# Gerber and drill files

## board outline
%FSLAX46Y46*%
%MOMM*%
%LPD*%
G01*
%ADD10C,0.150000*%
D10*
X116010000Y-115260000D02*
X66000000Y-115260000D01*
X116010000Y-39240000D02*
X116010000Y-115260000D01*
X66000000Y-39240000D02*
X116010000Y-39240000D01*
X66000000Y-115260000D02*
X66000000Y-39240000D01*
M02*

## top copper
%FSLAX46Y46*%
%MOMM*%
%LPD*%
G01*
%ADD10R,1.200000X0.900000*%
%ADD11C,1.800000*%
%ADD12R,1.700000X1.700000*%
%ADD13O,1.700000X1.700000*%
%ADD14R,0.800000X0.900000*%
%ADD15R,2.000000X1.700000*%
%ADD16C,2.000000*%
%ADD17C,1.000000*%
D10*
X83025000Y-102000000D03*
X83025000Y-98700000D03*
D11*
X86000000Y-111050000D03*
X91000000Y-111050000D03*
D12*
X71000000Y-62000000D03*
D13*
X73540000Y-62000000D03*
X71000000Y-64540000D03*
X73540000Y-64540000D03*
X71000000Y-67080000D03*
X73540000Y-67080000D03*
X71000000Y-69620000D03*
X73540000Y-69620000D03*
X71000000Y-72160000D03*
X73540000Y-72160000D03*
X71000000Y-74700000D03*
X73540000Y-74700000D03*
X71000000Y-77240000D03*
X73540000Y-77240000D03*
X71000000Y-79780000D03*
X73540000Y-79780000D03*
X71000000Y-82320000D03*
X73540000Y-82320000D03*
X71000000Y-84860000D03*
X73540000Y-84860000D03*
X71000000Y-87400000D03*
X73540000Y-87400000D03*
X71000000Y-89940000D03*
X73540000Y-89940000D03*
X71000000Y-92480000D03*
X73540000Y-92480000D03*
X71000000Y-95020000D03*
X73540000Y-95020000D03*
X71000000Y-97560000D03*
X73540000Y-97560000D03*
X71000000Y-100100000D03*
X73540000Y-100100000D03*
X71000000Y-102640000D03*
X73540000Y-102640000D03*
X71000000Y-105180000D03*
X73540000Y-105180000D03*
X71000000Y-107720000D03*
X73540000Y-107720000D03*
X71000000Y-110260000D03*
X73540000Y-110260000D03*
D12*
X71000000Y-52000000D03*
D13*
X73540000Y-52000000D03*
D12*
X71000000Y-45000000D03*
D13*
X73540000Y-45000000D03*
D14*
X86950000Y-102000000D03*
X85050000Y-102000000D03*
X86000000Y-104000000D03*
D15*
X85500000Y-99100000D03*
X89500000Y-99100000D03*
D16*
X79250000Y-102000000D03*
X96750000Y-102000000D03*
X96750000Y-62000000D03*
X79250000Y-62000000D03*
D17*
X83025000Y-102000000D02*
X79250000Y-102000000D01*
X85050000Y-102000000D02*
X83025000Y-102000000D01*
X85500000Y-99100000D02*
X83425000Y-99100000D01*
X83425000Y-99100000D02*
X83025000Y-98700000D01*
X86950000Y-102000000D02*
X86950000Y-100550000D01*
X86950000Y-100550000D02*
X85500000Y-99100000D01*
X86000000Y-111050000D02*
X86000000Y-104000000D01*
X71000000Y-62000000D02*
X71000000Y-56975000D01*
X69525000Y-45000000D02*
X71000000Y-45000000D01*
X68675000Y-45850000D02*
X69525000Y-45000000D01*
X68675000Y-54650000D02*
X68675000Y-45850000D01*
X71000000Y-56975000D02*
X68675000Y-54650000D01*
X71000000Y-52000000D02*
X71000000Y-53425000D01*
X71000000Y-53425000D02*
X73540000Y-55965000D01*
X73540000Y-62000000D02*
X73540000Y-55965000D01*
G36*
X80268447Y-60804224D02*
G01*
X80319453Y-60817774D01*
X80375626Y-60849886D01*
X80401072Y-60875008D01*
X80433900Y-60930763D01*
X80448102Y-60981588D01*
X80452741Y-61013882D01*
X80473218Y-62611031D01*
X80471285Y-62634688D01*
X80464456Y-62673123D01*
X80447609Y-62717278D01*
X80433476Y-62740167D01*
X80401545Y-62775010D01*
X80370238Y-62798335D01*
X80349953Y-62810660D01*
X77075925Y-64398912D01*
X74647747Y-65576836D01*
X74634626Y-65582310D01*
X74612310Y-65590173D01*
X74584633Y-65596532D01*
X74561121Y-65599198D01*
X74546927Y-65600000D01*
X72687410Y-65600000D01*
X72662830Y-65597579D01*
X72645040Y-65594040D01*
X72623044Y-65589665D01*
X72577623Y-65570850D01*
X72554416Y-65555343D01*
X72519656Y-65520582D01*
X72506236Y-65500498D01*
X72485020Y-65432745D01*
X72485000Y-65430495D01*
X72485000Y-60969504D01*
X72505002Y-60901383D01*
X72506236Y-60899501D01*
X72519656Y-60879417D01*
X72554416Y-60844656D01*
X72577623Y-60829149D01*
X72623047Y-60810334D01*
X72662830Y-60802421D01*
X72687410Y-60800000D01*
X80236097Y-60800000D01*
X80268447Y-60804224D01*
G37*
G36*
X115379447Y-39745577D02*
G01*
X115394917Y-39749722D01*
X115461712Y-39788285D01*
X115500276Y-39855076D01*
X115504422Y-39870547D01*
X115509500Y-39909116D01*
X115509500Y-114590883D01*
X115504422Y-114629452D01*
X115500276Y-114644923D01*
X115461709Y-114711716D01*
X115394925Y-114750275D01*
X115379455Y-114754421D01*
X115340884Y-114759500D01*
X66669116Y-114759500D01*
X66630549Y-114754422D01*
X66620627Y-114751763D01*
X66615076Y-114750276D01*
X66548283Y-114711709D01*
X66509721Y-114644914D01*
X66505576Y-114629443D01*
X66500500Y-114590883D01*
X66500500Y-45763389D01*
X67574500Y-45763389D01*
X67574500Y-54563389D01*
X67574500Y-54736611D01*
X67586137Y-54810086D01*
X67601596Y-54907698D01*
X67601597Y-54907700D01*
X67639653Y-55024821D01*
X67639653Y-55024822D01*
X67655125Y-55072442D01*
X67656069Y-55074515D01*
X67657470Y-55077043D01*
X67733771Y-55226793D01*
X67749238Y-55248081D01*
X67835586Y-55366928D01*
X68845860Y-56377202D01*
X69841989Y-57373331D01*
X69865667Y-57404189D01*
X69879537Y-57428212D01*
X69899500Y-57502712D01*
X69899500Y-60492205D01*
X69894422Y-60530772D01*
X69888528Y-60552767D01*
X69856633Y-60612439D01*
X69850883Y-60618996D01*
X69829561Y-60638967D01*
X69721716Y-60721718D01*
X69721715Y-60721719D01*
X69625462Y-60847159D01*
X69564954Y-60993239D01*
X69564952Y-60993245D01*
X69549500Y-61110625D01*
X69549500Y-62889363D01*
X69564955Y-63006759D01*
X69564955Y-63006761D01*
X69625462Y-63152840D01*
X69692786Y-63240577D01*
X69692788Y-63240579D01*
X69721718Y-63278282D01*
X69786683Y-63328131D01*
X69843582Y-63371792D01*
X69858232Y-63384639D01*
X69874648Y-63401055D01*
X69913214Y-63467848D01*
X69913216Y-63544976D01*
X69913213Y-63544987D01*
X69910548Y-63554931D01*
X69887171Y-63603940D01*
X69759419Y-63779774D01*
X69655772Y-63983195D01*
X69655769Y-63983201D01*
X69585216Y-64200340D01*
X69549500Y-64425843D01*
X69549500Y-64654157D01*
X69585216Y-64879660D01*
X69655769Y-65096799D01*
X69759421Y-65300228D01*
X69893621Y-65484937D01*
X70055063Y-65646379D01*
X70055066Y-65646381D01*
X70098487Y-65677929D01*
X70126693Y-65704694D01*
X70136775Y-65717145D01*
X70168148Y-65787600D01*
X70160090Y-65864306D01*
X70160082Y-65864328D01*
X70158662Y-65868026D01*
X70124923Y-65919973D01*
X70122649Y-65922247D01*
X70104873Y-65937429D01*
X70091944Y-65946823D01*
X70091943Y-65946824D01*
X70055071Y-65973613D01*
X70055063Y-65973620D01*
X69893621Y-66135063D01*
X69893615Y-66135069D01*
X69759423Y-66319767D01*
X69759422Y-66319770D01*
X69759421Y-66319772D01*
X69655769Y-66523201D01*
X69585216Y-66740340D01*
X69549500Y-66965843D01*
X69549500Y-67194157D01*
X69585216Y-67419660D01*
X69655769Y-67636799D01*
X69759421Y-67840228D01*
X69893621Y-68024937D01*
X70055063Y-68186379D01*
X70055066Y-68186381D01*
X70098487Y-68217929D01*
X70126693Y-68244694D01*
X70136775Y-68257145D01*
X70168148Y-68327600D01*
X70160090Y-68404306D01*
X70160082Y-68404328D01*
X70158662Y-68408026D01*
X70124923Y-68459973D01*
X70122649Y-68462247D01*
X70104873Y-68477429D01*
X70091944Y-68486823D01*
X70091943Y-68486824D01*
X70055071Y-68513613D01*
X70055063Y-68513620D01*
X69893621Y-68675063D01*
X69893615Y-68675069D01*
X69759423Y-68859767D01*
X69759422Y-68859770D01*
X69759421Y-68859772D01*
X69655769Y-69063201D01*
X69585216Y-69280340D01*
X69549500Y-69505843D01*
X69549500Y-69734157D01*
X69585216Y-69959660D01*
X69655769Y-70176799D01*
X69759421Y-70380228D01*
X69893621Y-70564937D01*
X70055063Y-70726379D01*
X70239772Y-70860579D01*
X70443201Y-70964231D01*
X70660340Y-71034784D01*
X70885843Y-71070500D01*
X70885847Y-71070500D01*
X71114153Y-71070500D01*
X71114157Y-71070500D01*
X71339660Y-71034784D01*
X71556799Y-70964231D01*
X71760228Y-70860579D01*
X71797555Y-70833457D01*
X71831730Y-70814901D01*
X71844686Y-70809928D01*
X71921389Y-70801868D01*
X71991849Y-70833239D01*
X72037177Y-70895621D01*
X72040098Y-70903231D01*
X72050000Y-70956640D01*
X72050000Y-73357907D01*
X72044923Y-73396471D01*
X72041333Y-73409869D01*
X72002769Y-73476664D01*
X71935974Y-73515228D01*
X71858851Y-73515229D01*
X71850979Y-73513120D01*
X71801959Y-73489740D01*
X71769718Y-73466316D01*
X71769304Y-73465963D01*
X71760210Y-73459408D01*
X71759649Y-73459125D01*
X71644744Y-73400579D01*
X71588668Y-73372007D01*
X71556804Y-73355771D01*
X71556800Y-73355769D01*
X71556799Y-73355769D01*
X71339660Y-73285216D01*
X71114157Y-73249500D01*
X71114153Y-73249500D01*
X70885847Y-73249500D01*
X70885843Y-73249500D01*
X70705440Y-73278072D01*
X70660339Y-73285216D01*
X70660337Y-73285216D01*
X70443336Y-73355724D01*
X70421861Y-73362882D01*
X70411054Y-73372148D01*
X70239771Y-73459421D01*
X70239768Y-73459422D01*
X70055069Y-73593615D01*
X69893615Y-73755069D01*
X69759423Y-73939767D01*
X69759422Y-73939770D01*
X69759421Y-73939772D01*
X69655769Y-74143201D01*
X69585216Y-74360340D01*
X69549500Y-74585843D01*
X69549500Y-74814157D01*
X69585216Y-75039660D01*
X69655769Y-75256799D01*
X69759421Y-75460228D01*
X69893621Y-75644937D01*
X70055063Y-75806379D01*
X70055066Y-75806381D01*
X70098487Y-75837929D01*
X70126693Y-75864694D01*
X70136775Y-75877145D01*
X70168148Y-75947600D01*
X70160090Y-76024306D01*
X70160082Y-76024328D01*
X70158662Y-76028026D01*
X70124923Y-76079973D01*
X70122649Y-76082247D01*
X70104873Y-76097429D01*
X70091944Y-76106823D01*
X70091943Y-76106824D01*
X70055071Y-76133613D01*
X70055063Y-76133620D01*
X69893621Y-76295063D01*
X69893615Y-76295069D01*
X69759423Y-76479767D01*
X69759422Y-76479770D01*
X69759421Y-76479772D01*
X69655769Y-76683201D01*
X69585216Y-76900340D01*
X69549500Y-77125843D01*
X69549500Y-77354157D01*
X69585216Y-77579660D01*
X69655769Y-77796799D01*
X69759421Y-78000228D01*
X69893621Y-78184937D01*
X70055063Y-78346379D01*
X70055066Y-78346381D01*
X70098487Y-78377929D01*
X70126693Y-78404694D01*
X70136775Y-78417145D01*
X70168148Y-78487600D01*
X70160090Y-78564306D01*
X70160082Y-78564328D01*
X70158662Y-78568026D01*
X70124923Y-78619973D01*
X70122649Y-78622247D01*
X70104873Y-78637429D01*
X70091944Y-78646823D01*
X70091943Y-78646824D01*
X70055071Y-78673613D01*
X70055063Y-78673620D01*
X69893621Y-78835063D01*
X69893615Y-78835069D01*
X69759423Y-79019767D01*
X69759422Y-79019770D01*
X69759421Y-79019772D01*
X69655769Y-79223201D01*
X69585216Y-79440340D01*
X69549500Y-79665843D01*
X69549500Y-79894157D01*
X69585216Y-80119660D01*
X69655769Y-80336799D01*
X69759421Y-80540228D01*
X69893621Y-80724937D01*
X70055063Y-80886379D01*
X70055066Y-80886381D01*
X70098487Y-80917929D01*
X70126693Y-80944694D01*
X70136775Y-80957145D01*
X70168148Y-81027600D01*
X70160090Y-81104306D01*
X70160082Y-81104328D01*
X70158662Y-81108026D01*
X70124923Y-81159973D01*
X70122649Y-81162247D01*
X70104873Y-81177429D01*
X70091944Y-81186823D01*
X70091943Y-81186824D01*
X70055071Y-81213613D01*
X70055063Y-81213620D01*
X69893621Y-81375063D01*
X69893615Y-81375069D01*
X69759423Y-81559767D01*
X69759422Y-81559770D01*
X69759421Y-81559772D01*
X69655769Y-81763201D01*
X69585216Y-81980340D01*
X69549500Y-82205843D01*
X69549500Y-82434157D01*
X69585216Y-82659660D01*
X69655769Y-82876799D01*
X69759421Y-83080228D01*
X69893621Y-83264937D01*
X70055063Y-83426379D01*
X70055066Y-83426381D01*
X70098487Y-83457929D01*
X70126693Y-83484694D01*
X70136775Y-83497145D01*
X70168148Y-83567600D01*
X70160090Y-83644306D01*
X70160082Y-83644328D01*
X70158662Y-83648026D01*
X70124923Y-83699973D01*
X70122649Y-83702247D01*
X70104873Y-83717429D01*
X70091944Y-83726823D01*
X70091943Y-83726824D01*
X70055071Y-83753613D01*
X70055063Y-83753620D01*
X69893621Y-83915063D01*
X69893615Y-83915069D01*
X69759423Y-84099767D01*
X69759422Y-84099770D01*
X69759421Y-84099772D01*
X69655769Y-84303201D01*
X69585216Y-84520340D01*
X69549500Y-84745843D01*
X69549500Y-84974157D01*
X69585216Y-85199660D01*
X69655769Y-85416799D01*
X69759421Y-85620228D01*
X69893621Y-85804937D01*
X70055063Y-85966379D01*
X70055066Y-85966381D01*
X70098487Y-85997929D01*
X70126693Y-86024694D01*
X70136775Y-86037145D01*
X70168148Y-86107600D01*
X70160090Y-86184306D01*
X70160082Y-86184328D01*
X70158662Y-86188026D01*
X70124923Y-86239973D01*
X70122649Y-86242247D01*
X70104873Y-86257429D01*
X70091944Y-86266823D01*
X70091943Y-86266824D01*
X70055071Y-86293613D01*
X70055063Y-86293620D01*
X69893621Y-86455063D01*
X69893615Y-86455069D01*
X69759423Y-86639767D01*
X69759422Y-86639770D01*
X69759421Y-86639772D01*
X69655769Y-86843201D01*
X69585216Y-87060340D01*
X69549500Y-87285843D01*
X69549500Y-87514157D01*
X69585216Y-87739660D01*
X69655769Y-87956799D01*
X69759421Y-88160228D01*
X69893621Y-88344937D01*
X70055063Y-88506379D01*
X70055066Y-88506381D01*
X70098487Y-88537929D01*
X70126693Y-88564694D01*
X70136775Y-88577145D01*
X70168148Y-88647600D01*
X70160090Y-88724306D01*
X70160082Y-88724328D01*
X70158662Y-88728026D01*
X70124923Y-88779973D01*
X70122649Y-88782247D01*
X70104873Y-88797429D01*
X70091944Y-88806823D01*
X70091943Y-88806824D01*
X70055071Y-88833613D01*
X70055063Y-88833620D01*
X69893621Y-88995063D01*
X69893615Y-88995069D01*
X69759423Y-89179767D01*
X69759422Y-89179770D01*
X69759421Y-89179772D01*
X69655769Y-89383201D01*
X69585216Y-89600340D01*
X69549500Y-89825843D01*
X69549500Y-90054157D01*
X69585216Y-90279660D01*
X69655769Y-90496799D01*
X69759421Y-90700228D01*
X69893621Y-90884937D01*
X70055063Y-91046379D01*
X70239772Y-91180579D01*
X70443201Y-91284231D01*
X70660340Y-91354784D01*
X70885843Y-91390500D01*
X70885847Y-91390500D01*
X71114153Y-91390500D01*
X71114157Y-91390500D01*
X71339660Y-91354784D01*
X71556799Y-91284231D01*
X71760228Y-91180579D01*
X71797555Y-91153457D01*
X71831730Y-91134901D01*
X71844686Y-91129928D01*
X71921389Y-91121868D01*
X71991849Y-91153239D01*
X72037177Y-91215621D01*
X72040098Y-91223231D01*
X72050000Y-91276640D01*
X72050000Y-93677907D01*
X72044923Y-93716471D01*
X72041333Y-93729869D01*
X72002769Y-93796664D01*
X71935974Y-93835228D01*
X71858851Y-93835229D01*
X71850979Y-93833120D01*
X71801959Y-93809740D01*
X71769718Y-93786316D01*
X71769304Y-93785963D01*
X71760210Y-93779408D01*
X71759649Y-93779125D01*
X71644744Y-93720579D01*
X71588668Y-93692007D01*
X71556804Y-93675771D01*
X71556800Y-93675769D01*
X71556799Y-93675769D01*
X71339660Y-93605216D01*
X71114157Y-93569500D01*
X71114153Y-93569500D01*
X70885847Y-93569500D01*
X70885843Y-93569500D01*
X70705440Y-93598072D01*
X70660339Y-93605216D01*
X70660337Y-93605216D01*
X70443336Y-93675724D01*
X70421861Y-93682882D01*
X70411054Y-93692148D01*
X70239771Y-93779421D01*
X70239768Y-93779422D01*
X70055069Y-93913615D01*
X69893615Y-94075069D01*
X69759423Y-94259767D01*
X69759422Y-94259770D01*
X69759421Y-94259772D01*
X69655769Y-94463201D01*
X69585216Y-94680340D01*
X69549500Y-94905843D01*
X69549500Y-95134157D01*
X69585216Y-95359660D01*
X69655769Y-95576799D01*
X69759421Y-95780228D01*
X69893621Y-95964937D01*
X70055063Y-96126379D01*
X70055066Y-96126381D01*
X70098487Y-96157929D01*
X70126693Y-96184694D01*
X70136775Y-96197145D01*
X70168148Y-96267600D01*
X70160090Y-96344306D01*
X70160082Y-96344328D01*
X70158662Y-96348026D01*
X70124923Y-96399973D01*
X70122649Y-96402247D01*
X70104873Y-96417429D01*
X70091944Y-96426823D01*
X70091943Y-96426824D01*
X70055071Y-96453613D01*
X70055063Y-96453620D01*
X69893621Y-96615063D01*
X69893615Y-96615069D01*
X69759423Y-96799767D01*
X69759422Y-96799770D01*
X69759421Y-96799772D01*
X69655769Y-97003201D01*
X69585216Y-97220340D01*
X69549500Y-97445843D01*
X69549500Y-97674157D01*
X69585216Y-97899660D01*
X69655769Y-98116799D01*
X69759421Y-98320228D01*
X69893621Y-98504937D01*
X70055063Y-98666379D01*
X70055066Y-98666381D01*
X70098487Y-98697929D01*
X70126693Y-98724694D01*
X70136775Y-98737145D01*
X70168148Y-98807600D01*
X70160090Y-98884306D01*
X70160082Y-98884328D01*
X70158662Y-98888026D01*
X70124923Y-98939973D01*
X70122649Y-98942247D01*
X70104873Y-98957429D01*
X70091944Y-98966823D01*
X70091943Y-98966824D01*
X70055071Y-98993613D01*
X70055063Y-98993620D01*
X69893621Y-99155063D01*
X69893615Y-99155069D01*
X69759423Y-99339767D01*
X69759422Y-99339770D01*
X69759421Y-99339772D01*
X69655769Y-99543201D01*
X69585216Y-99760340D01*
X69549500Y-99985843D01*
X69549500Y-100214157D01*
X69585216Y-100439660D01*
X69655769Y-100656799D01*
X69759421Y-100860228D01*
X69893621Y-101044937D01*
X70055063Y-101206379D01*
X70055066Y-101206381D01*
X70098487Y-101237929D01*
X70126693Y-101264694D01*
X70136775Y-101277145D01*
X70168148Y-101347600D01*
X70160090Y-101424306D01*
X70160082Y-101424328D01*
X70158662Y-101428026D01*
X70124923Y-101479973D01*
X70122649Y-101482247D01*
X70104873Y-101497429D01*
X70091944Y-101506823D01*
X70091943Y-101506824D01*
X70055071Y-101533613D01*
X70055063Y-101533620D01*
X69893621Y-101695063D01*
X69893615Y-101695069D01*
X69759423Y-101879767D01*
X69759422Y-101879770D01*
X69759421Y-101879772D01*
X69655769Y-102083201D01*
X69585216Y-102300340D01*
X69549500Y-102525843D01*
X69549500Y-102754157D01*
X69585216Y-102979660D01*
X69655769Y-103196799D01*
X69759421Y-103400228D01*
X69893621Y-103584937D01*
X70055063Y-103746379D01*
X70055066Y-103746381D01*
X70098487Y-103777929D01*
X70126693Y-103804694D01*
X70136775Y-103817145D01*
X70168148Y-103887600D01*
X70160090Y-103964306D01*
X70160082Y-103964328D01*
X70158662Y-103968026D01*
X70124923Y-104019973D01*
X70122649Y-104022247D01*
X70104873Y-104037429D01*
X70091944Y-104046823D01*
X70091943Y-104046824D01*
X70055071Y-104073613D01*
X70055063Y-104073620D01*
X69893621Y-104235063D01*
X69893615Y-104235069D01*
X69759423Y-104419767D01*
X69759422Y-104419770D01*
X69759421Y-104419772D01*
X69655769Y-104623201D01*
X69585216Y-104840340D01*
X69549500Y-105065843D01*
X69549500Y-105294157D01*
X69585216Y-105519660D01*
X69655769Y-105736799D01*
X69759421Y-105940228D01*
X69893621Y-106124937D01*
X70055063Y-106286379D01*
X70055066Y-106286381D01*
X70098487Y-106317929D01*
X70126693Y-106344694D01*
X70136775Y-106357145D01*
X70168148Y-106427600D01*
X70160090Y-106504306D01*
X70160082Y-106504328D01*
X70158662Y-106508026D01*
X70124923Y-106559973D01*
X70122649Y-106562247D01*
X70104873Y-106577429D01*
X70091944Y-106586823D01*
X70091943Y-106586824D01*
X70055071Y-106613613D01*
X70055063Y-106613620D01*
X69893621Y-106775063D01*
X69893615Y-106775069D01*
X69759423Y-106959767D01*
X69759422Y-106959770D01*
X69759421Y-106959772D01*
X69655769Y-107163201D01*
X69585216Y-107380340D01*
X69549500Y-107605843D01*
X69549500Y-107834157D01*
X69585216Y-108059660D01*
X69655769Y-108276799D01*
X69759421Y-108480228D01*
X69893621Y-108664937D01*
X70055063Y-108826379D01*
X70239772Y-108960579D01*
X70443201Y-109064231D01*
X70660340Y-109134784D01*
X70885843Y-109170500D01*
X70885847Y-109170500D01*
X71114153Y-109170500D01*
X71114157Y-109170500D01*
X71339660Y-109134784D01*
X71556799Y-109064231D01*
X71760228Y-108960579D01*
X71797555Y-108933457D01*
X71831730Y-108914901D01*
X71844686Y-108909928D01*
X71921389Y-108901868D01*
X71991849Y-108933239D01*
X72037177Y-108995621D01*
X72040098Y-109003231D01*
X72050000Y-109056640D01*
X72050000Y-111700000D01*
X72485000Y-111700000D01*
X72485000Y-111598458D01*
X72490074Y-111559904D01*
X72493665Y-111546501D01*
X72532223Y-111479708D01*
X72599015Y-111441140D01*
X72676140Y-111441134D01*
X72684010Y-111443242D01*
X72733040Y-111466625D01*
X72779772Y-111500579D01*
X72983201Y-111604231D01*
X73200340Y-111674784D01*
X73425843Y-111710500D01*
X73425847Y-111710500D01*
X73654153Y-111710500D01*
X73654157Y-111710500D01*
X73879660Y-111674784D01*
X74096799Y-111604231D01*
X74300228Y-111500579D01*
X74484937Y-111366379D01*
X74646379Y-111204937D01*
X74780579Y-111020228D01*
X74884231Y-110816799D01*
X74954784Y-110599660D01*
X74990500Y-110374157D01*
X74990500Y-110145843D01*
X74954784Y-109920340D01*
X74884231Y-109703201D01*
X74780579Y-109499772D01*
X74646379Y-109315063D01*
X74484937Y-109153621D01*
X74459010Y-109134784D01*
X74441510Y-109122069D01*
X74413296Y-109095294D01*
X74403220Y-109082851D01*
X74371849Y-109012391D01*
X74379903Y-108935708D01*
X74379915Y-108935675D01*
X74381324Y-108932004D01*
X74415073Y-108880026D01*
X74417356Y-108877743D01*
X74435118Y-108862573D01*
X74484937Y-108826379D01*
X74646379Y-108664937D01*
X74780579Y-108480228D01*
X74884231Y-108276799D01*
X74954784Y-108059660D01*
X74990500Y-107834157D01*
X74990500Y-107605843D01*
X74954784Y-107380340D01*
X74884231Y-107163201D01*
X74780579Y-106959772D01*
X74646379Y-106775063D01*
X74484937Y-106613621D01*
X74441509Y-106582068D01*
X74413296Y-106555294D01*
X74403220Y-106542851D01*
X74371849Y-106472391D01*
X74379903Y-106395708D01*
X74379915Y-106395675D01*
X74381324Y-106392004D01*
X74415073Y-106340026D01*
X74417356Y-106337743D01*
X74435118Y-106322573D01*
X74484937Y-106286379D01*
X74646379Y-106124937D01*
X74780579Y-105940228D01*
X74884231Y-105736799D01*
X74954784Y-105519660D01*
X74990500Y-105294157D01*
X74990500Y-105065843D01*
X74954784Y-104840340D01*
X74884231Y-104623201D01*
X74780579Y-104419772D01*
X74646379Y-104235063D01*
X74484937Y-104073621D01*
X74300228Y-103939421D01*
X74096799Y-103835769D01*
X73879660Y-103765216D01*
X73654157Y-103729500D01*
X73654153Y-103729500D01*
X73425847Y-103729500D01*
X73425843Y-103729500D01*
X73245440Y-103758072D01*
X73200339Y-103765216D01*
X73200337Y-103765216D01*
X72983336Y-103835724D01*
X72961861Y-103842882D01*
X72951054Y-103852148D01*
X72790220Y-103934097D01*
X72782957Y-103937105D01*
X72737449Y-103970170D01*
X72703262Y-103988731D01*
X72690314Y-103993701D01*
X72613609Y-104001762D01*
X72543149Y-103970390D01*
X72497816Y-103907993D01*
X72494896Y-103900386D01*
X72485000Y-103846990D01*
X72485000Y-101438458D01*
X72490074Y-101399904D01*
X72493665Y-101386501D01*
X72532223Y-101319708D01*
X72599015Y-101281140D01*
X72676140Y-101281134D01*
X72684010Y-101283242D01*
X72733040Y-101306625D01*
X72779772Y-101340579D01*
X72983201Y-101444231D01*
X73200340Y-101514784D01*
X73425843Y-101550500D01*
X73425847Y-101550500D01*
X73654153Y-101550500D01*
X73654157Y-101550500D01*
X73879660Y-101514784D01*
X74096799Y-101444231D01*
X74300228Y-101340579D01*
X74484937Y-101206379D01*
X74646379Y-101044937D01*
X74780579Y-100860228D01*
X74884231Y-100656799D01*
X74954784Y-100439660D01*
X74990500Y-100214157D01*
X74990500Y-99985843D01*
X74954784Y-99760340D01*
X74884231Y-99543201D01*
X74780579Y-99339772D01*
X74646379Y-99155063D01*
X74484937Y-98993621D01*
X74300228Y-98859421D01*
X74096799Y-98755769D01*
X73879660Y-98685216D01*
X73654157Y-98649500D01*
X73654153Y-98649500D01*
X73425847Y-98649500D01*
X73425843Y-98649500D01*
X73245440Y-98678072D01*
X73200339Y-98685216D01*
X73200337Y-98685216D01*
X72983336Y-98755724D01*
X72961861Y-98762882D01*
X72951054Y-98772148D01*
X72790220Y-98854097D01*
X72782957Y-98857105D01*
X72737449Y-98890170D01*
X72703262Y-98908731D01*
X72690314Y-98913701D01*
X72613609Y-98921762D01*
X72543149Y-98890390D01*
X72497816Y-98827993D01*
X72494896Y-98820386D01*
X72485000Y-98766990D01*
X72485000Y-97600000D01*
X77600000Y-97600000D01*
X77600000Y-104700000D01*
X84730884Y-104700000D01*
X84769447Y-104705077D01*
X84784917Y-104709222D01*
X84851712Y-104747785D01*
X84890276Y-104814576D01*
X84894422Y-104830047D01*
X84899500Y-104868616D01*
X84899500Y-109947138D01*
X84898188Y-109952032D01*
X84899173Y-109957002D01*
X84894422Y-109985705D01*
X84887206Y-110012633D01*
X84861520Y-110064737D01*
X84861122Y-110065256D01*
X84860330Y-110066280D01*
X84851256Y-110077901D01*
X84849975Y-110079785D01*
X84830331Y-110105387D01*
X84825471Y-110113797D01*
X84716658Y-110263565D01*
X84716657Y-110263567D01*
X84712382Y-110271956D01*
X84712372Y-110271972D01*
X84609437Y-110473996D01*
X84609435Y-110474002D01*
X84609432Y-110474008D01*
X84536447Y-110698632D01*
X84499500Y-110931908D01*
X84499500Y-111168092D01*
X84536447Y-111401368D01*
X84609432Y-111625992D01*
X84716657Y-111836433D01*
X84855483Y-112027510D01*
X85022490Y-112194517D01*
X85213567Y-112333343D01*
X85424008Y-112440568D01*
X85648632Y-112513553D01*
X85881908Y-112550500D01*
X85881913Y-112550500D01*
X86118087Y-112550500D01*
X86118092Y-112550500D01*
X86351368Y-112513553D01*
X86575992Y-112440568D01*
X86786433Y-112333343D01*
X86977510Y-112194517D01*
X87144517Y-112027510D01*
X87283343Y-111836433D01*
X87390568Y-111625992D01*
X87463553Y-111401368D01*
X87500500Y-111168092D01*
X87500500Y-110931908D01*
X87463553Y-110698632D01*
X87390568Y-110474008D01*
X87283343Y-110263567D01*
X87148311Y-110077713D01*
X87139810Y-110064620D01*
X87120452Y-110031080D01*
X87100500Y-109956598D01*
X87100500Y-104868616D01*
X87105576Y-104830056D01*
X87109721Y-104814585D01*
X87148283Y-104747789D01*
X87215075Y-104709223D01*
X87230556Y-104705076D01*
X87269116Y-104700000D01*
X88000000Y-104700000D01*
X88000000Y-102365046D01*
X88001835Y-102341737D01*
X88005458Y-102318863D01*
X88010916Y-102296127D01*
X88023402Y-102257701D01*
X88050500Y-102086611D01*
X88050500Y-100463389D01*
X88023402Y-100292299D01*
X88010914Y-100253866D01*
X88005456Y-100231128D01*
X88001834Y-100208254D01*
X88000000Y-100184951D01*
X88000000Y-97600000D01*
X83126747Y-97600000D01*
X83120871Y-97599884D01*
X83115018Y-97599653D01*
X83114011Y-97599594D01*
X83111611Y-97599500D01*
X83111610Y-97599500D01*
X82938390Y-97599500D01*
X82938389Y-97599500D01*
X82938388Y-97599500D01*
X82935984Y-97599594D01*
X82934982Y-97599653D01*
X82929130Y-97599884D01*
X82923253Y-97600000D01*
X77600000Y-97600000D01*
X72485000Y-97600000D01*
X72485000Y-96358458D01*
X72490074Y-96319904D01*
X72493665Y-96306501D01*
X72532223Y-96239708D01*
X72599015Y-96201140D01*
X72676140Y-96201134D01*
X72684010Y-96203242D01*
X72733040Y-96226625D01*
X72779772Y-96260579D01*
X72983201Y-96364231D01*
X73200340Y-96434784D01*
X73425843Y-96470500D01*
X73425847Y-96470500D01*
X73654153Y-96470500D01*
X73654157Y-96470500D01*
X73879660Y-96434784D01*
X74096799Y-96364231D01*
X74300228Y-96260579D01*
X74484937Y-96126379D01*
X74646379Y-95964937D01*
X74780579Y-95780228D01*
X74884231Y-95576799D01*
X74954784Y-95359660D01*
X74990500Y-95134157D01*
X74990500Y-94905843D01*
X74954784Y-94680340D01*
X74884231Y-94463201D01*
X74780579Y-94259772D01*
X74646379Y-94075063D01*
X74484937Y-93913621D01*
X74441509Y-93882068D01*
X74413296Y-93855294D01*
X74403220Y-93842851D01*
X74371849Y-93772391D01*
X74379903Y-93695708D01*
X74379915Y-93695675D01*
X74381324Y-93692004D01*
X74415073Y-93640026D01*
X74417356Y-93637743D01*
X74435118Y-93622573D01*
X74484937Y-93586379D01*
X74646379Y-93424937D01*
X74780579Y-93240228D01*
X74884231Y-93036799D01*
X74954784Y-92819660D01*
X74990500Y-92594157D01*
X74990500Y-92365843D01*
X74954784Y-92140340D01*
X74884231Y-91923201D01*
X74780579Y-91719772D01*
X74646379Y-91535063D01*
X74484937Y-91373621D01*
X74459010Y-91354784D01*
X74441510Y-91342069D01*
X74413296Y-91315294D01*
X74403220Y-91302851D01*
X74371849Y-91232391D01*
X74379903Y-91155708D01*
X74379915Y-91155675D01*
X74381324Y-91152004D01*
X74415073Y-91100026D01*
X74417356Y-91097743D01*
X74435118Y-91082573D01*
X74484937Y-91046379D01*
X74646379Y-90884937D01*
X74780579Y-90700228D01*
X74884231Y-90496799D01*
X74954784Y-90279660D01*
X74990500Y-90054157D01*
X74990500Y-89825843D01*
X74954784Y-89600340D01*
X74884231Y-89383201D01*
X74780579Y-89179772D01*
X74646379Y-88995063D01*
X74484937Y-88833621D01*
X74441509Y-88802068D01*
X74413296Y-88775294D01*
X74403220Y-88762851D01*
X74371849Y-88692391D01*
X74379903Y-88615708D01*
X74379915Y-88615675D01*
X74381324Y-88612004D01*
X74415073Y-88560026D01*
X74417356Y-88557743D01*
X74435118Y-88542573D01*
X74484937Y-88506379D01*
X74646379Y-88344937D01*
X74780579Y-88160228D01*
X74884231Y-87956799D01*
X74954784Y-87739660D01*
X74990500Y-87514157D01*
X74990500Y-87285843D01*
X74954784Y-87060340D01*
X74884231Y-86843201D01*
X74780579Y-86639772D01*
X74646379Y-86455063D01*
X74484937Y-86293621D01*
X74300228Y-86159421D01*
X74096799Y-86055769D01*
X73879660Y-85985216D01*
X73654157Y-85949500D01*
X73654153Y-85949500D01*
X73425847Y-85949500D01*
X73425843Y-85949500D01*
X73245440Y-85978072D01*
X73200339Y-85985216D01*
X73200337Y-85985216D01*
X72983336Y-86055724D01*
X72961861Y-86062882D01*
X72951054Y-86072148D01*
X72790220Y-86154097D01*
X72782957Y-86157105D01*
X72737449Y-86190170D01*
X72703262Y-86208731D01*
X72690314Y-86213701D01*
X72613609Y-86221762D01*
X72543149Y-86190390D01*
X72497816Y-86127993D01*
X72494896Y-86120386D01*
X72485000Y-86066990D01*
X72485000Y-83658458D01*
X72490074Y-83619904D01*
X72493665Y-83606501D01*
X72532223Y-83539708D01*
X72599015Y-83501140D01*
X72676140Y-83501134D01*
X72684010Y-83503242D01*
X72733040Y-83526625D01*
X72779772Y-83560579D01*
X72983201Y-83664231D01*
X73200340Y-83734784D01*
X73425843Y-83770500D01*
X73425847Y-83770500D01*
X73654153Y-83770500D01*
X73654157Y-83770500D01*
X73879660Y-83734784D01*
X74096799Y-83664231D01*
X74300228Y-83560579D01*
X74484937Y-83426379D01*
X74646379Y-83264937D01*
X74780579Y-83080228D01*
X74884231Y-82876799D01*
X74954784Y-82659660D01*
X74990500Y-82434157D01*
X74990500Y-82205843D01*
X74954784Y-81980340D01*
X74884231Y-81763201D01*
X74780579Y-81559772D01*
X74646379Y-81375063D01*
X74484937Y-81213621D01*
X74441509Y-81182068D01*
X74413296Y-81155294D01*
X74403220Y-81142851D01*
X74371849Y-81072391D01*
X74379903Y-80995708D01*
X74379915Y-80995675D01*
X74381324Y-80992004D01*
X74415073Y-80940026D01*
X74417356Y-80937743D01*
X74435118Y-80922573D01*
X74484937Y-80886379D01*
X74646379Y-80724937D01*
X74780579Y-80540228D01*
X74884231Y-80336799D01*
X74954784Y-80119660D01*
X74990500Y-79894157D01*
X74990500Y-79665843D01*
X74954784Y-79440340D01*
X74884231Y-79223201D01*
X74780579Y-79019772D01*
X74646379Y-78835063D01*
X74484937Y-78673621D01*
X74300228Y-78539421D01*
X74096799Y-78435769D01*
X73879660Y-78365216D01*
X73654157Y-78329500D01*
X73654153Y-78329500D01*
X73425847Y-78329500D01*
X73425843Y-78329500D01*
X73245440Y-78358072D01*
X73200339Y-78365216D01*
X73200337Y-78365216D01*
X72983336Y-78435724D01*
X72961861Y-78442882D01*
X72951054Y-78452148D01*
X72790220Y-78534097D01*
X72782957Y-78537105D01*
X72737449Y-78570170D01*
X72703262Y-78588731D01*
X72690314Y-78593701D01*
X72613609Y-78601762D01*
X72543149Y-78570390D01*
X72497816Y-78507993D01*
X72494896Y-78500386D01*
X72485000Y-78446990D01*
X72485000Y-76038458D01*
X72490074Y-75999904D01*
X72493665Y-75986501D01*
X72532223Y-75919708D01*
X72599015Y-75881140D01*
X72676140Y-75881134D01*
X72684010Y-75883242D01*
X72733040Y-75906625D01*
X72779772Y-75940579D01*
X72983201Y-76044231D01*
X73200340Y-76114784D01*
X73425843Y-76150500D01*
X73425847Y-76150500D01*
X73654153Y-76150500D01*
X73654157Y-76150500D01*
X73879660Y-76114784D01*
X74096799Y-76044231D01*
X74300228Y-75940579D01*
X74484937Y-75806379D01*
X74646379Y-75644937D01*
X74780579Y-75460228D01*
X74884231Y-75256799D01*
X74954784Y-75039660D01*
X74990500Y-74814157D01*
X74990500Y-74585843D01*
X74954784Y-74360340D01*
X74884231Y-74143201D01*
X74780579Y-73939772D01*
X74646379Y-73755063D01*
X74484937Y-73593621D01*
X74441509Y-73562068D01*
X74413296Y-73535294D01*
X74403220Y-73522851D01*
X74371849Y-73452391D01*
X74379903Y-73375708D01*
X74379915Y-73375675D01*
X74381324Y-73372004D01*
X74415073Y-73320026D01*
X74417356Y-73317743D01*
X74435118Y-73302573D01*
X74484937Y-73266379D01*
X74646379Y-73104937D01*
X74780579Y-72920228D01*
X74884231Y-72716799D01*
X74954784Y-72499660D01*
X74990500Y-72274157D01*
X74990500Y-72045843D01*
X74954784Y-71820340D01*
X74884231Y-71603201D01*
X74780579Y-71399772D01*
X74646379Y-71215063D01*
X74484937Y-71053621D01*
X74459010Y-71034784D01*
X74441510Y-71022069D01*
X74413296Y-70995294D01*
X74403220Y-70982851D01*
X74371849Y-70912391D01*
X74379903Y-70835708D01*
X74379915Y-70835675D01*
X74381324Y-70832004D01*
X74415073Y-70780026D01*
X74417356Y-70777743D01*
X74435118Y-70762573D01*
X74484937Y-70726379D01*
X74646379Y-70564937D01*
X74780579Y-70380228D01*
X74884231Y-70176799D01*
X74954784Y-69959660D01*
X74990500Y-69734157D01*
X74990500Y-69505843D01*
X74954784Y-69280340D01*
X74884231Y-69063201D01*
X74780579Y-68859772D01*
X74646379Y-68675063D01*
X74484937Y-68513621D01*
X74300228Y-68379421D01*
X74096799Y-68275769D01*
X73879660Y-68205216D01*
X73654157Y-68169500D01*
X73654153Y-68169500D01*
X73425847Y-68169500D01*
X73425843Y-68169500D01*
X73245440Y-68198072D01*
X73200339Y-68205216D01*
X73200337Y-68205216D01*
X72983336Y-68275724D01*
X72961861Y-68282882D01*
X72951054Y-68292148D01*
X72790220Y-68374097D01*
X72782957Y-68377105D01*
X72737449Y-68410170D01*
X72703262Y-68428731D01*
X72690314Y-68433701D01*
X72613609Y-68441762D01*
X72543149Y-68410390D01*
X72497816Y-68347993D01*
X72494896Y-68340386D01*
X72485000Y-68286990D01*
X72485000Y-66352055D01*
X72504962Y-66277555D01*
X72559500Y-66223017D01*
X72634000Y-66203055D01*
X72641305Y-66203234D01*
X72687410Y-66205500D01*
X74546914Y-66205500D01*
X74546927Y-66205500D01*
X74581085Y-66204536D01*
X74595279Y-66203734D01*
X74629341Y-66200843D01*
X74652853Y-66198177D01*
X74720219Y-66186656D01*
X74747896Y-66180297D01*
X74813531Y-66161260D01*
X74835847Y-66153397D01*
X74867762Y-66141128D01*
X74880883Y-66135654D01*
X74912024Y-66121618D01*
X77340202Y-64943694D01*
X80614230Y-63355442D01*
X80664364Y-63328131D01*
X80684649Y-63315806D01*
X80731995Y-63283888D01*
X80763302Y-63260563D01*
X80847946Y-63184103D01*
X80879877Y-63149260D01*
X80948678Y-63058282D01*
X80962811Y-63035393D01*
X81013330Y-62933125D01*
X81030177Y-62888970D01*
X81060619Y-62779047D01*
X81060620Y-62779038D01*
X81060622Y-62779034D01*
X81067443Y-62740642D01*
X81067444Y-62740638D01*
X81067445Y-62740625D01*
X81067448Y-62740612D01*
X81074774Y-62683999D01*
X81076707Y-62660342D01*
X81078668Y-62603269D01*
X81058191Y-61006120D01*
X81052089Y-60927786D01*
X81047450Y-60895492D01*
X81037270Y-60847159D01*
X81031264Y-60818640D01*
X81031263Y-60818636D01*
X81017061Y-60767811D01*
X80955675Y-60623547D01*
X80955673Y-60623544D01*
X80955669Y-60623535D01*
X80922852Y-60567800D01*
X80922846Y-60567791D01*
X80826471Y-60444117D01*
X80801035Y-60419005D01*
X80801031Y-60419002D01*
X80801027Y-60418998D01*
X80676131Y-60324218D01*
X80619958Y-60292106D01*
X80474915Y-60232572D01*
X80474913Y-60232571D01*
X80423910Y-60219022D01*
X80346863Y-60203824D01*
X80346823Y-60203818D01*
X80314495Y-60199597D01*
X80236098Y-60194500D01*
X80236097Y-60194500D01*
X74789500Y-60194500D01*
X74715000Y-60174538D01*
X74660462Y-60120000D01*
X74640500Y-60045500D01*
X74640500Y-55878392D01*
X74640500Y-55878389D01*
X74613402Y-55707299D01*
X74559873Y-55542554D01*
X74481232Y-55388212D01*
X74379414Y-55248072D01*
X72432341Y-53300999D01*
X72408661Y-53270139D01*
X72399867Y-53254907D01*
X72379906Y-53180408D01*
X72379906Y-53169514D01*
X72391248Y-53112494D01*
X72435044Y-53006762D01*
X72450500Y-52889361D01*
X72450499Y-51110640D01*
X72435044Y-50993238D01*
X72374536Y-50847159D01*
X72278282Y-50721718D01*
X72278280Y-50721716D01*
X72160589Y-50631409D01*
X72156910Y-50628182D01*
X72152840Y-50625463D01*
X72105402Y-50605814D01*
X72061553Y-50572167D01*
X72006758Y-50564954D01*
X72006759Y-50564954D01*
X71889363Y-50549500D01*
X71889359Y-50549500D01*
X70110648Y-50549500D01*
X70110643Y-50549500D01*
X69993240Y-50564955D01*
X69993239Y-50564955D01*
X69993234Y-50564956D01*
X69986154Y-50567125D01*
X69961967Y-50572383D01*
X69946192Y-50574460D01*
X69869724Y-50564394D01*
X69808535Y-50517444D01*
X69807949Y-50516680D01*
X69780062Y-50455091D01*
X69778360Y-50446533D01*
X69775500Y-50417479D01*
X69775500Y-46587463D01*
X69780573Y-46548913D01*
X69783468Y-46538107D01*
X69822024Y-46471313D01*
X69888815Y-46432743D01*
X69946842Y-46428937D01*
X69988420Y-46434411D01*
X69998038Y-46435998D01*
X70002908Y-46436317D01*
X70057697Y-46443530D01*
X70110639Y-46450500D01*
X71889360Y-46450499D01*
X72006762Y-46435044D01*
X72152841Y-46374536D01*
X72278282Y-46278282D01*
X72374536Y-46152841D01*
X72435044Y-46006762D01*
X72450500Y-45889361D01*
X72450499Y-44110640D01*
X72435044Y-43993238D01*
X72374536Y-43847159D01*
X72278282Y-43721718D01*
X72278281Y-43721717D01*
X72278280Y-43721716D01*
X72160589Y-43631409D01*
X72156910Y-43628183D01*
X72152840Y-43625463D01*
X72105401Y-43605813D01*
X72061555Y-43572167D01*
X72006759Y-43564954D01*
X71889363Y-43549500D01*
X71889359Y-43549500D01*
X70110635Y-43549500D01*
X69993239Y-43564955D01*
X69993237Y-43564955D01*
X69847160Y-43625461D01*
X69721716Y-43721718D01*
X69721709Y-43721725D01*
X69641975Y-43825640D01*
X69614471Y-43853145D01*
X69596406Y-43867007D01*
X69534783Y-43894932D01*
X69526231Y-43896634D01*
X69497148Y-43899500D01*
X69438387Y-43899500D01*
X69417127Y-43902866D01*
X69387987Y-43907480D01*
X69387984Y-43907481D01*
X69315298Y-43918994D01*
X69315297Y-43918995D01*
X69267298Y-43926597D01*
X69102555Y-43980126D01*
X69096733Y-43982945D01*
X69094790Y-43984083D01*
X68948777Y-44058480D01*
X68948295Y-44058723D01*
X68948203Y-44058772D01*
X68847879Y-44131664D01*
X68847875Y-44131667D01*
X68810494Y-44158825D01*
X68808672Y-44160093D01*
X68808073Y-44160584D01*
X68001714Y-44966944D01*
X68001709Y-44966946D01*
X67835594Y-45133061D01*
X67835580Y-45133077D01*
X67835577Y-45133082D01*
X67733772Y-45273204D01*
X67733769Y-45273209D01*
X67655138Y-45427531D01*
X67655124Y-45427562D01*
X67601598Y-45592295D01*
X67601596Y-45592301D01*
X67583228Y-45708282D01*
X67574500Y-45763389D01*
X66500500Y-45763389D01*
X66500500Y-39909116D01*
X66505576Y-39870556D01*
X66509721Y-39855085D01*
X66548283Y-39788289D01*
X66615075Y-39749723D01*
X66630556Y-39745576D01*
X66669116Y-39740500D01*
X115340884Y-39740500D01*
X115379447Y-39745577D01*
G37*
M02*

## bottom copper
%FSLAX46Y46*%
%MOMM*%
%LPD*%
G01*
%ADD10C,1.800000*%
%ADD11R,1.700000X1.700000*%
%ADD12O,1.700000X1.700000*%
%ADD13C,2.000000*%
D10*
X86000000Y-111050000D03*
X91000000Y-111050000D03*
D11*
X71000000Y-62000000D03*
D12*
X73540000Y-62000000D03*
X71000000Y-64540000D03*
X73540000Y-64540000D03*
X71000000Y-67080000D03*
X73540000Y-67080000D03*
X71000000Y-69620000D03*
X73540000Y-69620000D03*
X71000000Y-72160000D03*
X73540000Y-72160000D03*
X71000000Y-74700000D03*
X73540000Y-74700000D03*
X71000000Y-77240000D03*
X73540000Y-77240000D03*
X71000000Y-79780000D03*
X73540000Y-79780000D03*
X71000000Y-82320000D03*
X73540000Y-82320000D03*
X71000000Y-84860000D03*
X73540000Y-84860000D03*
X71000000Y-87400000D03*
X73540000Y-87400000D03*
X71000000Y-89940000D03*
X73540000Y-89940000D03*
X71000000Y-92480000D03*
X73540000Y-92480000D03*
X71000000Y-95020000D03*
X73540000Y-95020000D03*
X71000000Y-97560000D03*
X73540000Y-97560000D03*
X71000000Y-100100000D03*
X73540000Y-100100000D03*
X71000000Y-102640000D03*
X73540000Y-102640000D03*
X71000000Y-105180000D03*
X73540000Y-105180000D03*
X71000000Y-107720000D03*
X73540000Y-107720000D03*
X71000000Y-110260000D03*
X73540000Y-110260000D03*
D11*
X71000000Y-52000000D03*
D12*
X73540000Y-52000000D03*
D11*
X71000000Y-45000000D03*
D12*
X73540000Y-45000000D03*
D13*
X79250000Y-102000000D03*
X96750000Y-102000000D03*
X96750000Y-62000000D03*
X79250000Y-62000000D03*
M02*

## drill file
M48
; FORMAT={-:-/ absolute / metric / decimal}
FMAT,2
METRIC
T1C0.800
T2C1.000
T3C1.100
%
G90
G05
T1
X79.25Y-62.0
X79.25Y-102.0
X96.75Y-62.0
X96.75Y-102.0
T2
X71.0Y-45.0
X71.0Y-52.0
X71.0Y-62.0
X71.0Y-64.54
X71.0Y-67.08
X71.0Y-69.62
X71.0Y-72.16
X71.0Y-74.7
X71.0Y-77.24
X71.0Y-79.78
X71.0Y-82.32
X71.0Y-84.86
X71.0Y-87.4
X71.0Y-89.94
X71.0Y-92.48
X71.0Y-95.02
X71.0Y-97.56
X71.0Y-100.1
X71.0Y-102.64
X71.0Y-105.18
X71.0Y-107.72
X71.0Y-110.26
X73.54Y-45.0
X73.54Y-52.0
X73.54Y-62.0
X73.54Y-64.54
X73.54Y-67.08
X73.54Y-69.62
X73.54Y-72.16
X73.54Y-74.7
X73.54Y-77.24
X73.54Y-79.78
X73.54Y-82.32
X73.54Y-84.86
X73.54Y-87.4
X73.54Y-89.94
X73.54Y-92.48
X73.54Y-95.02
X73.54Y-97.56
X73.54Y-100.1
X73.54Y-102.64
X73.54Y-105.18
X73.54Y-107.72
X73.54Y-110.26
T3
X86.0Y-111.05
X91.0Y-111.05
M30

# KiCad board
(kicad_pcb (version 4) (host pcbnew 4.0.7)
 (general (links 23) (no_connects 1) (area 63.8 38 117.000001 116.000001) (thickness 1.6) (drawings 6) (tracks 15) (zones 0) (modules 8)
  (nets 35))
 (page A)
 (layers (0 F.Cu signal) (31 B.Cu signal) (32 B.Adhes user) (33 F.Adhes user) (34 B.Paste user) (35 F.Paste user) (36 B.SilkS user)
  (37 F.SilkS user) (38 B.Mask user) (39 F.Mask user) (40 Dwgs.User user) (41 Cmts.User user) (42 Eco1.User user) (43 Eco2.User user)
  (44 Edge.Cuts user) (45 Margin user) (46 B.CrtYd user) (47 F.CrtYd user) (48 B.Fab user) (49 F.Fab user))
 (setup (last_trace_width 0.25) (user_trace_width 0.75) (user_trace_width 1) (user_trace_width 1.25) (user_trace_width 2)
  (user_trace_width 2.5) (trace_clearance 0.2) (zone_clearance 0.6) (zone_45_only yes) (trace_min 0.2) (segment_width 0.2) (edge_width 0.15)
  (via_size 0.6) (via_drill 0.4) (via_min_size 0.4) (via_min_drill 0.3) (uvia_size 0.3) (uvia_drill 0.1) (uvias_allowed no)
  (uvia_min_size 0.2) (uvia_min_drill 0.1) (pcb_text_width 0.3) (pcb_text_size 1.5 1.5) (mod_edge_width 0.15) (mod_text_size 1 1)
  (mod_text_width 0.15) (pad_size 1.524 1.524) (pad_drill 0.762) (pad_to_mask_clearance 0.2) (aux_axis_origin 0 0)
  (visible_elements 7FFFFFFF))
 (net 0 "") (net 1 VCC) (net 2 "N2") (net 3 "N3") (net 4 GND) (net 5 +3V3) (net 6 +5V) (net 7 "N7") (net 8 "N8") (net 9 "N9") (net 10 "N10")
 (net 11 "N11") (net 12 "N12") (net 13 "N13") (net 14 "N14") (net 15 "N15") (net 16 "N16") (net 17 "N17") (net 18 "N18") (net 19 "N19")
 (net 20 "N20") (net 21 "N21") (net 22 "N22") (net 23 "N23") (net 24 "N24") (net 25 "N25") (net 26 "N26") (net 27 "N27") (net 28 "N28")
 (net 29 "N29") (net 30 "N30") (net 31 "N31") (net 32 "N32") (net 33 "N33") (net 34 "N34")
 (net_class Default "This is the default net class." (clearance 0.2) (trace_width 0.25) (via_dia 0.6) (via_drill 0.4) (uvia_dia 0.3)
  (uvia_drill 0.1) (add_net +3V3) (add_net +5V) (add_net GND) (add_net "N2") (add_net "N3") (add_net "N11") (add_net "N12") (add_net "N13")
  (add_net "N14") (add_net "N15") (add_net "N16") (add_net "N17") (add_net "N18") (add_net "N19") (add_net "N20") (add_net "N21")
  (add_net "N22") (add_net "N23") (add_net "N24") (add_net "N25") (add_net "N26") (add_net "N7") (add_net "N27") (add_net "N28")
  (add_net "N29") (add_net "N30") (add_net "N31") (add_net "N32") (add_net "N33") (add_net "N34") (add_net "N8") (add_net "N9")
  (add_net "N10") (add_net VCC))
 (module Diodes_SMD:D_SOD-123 (layer F.Cu) (at 83.025 100.35 90)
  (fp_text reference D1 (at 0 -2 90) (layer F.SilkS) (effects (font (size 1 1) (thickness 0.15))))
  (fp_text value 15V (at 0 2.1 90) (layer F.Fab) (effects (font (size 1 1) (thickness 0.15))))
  (pad 1 smd rect (at -1.65 0 90) (size 0.9 1.2) (layers F.Cu F.Paste F.Mask) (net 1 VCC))
  (pad 2 smd rect (at 1.65 0 90) (size 0.9 1.2) (layers F.Cu F.Paste F.Mask) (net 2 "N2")))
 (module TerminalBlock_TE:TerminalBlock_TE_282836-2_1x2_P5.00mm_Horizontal (layer F.Cu) (at 86 111.05)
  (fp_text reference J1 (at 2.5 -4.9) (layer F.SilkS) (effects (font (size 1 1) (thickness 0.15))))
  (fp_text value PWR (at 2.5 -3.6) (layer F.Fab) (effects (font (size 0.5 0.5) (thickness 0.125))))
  (pad 1 thru_hole circle (at 0 0) (size 1.8 1.8) (drill 1.1) (layers *.Cu *.Mask) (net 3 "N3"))
  (pad 2 thru_hole circle (at 5 0) (size 1.8 1.8) (drill 1.1) (layers *.Cu *.Mask) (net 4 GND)))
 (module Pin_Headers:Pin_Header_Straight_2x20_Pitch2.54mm (layer F.Cu) (at 71 62)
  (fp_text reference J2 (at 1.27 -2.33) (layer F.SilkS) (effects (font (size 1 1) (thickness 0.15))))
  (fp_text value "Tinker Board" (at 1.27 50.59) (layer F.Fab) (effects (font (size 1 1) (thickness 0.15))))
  (pad 1 thru_hole rect (at 0 0) (size 1.7 1.7) (drill 1) (layers *.Cu *.Mask) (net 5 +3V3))
  (pad 2 thru_hole oval (at 2.54 0) (size 1.7 1.7) (drill 1) (layers *.Cu *.Mask) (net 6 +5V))
  (pad 3 thru_hole oval (at 0 2.54) (size 1.7 1.7) (drill 1) (layers *.Cu *.Mask) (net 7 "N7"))
  (pad 4 thru_hole oval (at 2.54 2.54) (size 1.7 1.7) (drill 1) (layers *.Cu *.Mask) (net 6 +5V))
  (pad 5 thru_hole oval (at 0 5.08) (size 1.7 1.7) (drill 1) (layers *.Cu *.Mask) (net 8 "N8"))
  (pad 6 thru_hole oval (at 2.54 5.08) (size 1.7 1.7) (drill 1) (layers *.Cu *.Mask) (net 4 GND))
  (pad 7 thru_hole oval (at 0 7.62) (size 1.7 1.7) (drill 1) (layers *.Cu *.Mask) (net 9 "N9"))
  (pad 8 thru_hole oval (at 2.54 7.62) (size 1.7 1.7) (drill 1) (layers *.Cu *.Mask) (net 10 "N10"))
  (pad 9 thru_hole oval (at 0 10.16) (size 1.7 1.7) (drill 1) (layers *.Cu *.Mask) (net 4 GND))
  (pad 10 thru_hole oval (at 2.54 10.16) (size 1.7 1.7) (drill 1) (layers *.Cu *.Mask) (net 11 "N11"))
  (pad 11 thru_hole oval (at 0 12.7) (size 1.7 1.7) (drill 1) (layers *.Cu *.Mask) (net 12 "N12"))
  (pad 12 thru_hole oval (at 2.54 12.7) (size 1.7 1.7) (drill 1) (layers *.Cu *.Mask) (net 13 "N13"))
  (pad 13 thru_hole oval (at 0 15.24) (size 1.7 1.7) (drill 1) (layers *.Cu *.Mask) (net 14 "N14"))
  (pad 14 thru_hole oval (at 2.54 15.24) (size 1.7 1.7) (drill 1) (layers *.Cu *.Mask) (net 4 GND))
  (pad 15 thru_hole oval (at 0 17.78) (size 1.7 1.7) (drill 1) (layers *.Cu *.Mask) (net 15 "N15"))
  (pad 16 thru_hole oval (at 2.54 17.78) (size 1.7 1.7) (drill 1) (layers *.Cu *.Mask) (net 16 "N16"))
  (pad 17 thru_hole oval (at 0 20.32) (size 1.7 1.7) (drill 1) (layers *.Cu *.Mask) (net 5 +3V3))
  (pad 18 thru_hole oval (at 2.54 20.32) (size 1.7 1.7) (drill 1) (layers *.Cu *.Mask) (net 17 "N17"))
  (pad 19 thru_hole oval (at 0 22.86) (size 1.7 1.7) (drill 1) (layers *.Cu *.Mask) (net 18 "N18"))
  (pad 20 thru_hole oval (at 2.54 22.86) (size 1.7 1.7) (drill 1) (layers *.Cu *.Mask) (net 4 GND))
  (pad 21 thru_hole oval (at 0 25.4) (size 1.7 1.7) (drill 1) (layers *.Cu *.Mask) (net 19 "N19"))
  (pad 22 thru_hole oval (at 2.54 25.4) (size 1.7 1.7) (drill 1) (layers *.Cu *.Mask) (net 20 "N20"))
  (pad 23 thru_hole oval (at 0 27.94) (size 1.7 1.7) (drill 1) (layers *.Cu *.Mask) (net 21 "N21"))
  (pad 24 thru_hole oval (at 2.54 27.94) (size 1.7 1.7) (drill 1) (layers *.Cu *.Mask) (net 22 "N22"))
  (pad 25 thru_hole oval (at 0 30.48) (size 1.7 1.7) (drill 1) (layers *.Cu *.Mask) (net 4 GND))
  (pad 26 thru_hole oval (at 2.54 30.48) (size 1.7 1.7) (drill 1) (layers *.Cu *.Mask) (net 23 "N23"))
  (pad 27 thru_hole oval (at 0 33.02) (size 1.7 1.7) (drill 1) (layers *.Cu *.Mask) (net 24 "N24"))
  (pad 28 thru_hole oval (at 2.54 33.02) (size 1.7 1.7) (drill 1) (layers *.Cu *.Mask) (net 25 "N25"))
  (pad 29 thru_hole oval (at 0 35.56) (size 1.7 1.7) (drill 1) (layers *.Cu *.Mask) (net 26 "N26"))
  (pad 30 thru_hole oval (at 2.54 35.56) (size 1.7 1.7) (drill 1) (layers *.Cu *.Mask) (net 4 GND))
  (pad 31 thru_hole oval (at 0 38.1) (size 1.7 1.7) (drill 1) (layers *.Cu *.Mask) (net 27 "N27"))
  (pad 32 thru_hole oval (at 2.54 38.1) (size 1.7 1.7) (drill 1) (layers *.Cu *.Mask) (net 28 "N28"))
  (pad 33 thru_hole oval (at 0 40.64) (size 1.7 1.7) (drill 1) (layers *.Cu *.Mask) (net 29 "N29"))
  (pad 34 thru_hole oval (at 2.54 40.64) (size 1.7 1.7) (drill 1) (layers *.Cu *.Mask) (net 4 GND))
  (pad 35 thru_hole oval (at 0 43.18) (size 1.7 1.7) (drill 1) (layers *.Cu *.Mask) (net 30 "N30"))
  (pad 36 thru_hole oval (at 2.54 43.18) (size 1.7 1.7) (drill 1) (layers *.Cu *.Mask) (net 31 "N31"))
  (pad 37 thru_hole oval (at 0 45.72) (size 1.7 1.7) (drill 1) (layers *.Cu *.Mask) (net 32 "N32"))
  (pad 38 thru_hole oval (at 2.54 45.72) (size 1.7 1.7) (drill 1) (layers *.Cu *.Mask) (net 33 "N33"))
  (pad 39 thru_hole oval (at 0 48.26) (size 1.7 1.7) (drill 1) (layers *.Cu *.Mask) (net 4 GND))
  (pad 40 thru_hole oval (at 2.54 48.26) (size 1.7 1.7) (drill 1) (layers *.Cu *.Mask) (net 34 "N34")))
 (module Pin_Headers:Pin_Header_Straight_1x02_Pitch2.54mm (layer F.Cu) (at 71 52 90)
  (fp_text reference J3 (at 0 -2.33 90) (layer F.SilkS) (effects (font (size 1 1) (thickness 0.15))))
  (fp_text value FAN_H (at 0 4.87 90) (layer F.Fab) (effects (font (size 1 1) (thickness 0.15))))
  (pad 1 thru_hole rect (at 0 0 90) (size 1.7 1.7) (drill 1) (layers *.Cu *.Mask) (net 6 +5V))
  (pad 2 thru_hole oval (at 0 2.54 90) (size 1.7 1.7) (drill 1) (layers *.Cu *.Mask) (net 4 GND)))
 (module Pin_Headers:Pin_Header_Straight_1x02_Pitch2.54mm (layer F.Cu) (at 71 45 90)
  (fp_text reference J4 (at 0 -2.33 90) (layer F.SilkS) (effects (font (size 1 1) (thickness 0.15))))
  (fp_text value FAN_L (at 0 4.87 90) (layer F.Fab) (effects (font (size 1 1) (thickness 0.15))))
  (pad 1 thru_hole rect (at 0 0 90) (size 1.7 1.7) (drill 1) (layers *.Cu *.Mask) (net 5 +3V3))
  (pad 2 thru_hole oval (at 0 2.54 90) (size 1.7 1.7) (drill 1) (layers *.Cu *.Mask) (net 4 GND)))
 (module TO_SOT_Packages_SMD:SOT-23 (layer F.Cu) (at 86 103 270)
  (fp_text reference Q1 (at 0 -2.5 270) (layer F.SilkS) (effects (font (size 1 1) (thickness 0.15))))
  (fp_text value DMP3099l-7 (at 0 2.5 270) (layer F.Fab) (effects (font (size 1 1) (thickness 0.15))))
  (pad 1 smd rect (at -1 -0.95 270) (size 0.9 0.8) (layers F.Cu F.Paste F.Mask) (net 2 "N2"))
  (pad 2 smd rect (at -1 0.95 270) (size 0.9 0.8) (layers F.Cu F.Paste F.Mask) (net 1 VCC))
  (pad 3 smd rect (at 1 0 270) (size 0.9 0.8) (layers F.Cu F.Paste F.Mask) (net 3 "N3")))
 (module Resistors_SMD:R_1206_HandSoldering (layer F.Cu) (at 87.5 99.1)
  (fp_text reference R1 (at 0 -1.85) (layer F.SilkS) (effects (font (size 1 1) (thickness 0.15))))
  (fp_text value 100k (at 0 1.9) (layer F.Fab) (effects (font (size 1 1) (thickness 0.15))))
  (pad 1 smd rect (at -2 0) (size 2 1.7) (layers F.Cu F.Paste F.Mask) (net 2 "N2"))
  (pad 2 smd rect (at 2 0) (size 2 1.7) (layers F.Cu F.Paste F.Mask) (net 4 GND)))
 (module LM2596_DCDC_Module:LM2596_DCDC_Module (layer F.Cu) (at 88 82 90)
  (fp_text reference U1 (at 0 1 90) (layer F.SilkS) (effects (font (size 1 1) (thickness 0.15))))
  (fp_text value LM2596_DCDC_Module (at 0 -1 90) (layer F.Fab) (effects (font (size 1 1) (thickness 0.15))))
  (pad 1 thru_hole circle (at -20 -8.75 90) (size 2 2) (drill 0.8) (layers *.Cu *.Mask) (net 1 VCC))
  (pad 2 thru_hole circle (at -20 8.75 90) (size 2 2) (drill 0.8) (layers *.Cu *.Mask) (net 4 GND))
  (pad 3 thru_hole circle (at 20 8.75 90) (size 2 2) (drill 0.8) (layers *.Cu *.Mask) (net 4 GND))
  (pad 4 thru_hole circle (at 20 -8.75 90) (size 2 2) (drill 0.8) (layers *.Cu *.Mask) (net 6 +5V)))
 (gr_line (start 116.01 115.26) (end 66 115.26) (angle 90) (layer Edge.Cuts) (width 0.15))
 (gr_line (start 116.01 39.24) (end 116.01 115.26) (angle 90) (layer Edge.Cuts) (width 0.15))
 (gr_line (start 66 39.24) (end 116.01 39.24) (angle 90) (layer Edge.Cuts) (width 0.15))
 (gr_line (start 66 115.26) (end 66 39.24) (angle 90) (layer Edge.Cuts) (width 0.15))
 (segment (start 83.025 102) (end 79.25 102) (width 1) (layer F.Cu) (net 1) (status 30))
 (segment (start 85.05 102) (end 83.025 102) (width 1) (layer F.Cu) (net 1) (status 30))
 (segment (start 85.5 99.1) (end 83.425 99.1) (width 1) (layer F.Cu) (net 2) (status 30))
 (segment (start 83.425 99.1) (end 83.025 98.7) (width 1) (layer F.Cu) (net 2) (status 30))
 (segment (start 86.95 102) (end 86.95 100.55) (width 1) (layer F.Cu) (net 2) (status 10))
 (segment (start 86.95 100.55) (end 85.5 99.1) (width 1) (layer F.Cu) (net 2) (status 20))
 (segment (start 86 111.05) (end 86 104) (width 1) (layer F.Cu) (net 3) (status 30))
 (segment (start 71 62) (end 71 56.975) (width 1) (layer F.Cu) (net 5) (status 10))
 (segment (start 69.525 45) (end 71 45) (width 1) (layer F.Cu) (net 5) (status 20))
 (segment (start 68.675 45.85) (end 69.525 45) (width 1) (layer F.Cu) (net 5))
 (segment (start 68.675 54.65) (end 68.675 45.85) (width 1) (layer F.Cu) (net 5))
 (segment (start 71 56.975) (end 68.675 54.65) (width 1) (layer F.Cu) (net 5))
 (segment (start 71 52) (end 71 53.425) (width 1) (layer F.Cu) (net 6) (status 10))
 (segment (start 71 53.425) (end 73.54 55.965) (width 1) (layer F.Cu) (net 6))
 (segment (start 73.54 62) (end 73.54 55.965) (width 1) (layer F.Cu) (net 6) (status 10))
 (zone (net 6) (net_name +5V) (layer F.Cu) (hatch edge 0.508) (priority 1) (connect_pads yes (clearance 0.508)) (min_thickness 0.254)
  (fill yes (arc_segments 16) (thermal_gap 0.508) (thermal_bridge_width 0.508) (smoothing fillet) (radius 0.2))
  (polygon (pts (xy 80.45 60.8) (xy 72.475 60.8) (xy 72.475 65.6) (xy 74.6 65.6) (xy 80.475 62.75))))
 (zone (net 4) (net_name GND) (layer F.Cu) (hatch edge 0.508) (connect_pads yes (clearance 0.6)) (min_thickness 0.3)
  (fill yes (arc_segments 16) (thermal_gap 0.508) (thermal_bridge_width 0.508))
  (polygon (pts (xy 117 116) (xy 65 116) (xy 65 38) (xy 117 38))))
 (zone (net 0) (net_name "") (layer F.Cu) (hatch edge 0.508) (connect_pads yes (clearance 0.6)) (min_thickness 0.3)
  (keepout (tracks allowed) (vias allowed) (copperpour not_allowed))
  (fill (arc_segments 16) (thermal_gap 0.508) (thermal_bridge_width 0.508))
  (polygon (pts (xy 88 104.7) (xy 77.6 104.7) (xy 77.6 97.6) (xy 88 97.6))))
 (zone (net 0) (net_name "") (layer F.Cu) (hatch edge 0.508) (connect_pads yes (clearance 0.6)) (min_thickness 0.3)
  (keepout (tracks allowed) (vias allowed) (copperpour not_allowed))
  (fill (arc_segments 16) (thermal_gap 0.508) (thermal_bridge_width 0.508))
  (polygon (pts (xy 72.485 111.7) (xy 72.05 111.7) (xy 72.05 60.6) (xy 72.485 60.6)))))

